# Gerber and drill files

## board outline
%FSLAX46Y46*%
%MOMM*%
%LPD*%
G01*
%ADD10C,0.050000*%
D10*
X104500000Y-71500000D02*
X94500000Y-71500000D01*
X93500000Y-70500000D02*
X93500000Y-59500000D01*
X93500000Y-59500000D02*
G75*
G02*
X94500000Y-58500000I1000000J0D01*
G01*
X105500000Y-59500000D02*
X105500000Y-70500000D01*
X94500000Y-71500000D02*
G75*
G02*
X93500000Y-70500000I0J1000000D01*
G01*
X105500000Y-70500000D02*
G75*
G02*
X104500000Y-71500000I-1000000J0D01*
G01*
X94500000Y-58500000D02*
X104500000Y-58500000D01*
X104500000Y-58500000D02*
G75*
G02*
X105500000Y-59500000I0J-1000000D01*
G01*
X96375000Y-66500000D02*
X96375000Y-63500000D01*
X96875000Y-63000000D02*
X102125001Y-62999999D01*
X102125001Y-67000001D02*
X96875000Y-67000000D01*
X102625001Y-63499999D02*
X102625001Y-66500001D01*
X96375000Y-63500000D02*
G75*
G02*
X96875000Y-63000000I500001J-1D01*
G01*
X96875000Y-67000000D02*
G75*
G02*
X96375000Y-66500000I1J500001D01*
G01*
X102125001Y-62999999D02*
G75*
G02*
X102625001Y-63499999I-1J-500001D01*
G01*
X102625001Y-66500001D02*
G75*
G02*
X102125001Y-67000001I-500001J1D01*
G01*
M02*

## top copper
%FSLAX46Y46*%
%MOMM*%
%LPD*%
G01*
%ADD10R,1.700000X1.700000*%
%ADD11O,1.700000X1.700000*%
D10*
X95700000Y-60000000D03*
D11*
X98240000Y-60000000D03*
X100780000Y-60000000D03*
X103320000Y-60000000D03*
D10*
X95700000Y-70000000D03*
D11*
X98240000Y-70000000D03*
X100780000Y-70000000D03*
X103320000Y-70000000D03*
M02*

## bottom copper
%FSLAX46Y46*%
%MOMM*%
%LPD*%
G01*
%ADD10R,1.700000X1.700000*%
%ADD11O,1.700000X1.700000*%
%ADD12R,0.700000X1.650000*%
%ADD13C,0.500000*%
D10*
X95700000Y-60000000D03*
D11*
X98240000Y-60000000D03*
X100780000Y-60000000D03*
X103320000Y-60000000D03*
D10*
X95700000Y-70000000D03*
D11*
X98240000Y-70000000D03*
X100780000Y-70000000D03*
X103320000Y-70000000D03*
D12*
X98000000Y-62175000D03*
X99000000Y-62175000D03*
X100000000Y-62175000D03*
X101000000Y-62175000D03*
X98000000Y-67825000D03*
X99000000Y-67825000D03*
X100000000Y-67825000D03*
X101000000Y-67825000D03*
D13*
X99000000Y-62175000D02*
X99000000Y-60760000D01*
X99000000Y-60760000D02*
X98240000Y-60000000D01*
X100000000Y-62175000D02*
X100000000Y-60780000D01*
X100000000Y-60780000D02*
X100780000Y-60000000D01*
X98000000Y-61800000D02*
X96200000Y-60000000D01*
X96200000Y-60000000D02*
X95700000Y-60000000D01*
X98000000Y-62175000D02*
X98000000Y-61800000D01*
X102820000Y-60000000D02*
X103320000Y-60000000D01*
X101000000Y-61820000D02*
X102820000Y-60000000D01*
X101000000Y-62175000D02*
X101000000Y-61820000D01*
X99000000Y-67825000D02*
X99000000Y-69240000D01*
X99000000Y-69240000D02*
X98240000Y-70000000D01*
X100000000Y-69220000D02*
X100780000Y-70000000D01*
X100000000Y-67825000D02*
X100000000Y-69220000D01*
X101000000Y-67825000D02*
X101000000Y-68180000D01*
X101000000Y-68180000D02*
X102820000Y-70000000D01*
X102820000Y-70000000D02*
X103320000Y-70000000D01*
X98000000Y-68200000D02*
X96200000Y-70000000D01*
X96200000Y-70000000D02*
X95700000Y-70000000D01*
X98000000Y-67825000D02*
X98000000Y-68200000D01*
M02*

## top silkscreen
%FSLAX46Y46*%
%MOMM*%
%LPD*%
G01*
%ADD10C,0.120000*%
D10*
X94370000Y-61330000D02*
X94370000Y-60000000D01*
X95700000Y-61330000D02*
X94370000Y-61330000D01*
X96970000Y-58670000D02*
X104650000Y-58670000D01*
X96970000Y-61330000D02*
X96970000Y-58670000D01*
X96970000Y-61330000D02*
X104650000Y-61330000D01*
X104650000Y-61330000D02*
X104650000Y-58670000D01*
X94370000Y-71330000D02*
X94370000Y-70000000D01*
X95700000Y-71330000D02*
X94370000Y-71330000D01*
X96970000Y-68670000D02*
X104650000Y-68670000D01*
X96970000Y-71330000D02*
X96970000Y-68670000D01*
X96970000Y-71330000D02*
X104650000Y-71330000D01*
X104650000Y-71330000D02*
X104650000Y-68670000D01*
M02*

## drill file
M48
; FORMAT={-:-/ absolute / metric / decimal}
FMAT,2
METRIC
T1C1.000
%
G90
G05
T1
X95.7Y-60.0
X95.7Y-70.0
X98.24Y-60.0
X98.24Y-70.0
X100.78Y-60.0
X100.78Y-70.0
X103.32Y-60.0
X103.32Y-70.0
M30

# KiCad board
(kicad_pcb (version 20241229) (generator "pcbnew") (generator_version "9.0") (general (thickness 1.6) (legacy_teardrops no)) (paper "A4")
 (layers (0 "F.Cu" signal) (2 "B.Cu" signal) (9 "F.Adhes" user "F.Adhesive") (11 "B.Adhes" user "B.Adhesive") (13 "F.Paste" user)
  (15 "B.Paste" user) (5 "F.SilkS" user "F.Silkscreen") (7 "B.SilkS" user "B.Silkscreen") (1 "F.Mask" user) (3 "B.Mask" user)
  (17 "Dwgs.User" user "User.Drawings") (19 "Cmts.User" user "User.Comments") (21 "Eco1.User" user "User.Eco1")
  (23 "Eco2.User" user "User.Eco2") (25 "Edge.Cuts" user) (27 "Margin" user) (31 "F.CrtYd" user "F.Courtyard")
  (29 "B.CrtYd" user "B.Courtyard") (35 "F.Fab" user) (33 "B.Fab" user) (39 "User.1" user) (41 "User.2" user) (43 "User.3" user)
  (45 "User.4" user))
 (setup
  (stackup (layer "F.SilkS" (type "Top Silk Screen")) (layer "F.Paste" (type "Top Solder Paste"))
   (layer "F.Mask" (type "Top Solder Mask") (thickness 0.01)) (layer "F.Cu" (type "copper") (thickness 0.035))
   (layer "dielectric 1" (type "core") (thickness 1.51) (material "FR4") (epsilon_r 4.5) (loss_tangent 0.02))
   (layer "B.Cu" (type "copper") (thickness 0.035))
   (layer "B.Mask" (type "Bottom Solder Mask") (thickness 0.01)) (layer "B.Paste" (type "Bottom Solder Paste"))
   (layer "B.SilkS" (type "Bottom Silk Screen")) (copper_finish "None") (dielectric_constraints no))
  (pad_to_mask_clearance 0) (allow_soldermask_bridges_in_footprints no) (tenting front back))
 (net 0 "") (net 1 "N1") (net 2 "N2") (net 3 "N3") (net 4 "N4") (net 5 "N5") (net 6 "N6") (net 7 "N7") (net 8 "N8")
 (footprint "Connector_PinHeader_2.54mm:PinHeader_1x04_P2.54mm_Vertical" (layer "F.Cu") (at 95.7 60 90)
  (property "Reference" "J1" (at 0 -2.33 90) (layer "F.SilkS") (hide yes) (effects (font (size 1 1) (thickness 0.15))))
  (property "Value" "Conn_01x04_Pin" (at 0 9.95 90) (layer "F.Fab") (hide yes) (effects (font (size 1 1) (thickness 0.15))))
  (fp_line (start -1.33 -1.33) (end 0 -1.33) (stroke (width 0.12) (type solid)) (layer "F.SilkS"))
  (fp_line (start -1.33 0) (end -1.33 -1.33) (stroke (width 0.12) (type solid)) (layer "F.SilkS"))
  (fp_line (start 1.33 1.27) (end 1.33 8.95) (stroke (width 0.12) (type solid)) (layer "F.SilkS"))
  (fp_line (start -1.33 1.27) (end 1.33 1.27) (stroke (width 0.12) (type solid)) (layer "F.SilkS"))
  (fp_line (start -1.33 1.27) (end -1.33 8.95) (stroke (width 0.12) (type solid)) (layer "F.SilkS"))
  (fp_line (start -1.33 8.95) (end 1.33 8.95) (stroke (width 0.12) (type solid)) (layer "F.SilkS"))
  (pad "1" thru_hole rect (at 0 0 90) (size 1.7 1.7) (drill 1) (layers "*.Cu" "*.Mask") (remove_unused_layers no) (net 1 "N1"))
  (pad "2" thru_hole oval (at 0 2.54 90) (size 1.7 1.7) (drill 1) (layers "*.Cu" "*.Mask") (remove_unused_layers no) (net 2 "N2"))
  (pad "3" thru_hole oval (at 0 5.08 90) (size 1.7 1.7) (drill 1) (layers "*.Cu" "*.Mask") (remove_unused_layers no) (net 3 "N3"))
  (pad "4" thru_hole oval (at 0 7.62 90) (size 1.7 1.7) (drill 1) (layers "*.Cu" "*.Mask") (remove_unused_layers no) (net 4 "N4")))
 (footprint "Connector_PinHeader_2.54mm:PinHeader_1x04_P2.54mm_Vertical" (layer "F.Cu") (at 95.7 70 90)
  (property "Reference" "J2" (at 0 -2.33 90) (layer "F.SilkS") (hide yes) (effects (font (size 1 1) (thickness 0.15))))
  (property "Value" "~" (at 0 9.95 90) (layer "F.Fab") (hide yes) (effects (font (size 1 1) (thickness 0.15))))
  (fp_line (start -1.33 -1.33) (end 0 -1.33) (stroke (width 0.12) (type solid)) (layer "F.SilkS"))
  (fp_line (start -1.33 0) (end -1.33 -1.33) (stroke (width 0.12) (type solid)) (layer "F.SilkS"))
  (fp_line (start 1.33 1.27) (end 1.33 8.95) (stroke (width 0.12) (type solid)) (layer "F.SilkS"))
  (fp_line (start -1.33 1.27) (end 1.33 1.27) (stroke (width 0.12) (type solid)) (layer "F.SilkS"))
  (fp_line (start -1.33 1.27) (end -1.33 8.95) (stroke (width 0.12) (type solid)) (layer "F.SilkS"))
  (fp_line (start -1.33 8.95) (end 1.33 8.95) (stroke (width 0.12) (type solid)) (layer "F.SilkS"))
  (pad "1" thru_hole rect (at 0 0 90) (size 1.7 1.7) (drill 1) (layers "*.Cu" "*.Mask") (remove_unused_layers no) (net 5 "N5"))
  (pad "2" thru_hole oval (at 0 2.54 90) (size 1.7 1.7) (drill 1) (layers "*.Cu" "*.Mask") (remove_unused_layers no) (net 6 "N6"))
  (pad "3" thru_hole oval (at 0 5.08 90) (size 1.7 1.7) (drill 1) (layers "*.Cu" "*.Mask") (remove_unused_layers no) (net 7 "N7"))
  (pad "4" thru_hole oval (at 0 7.62 90) (size 1.7 1.7) (drill 1) (layers "*.Cu" "*.Mask") (remove_unused_layers no) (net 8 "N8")))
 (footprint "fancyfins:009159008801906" (layer "B.Cu") (at 99.5 65)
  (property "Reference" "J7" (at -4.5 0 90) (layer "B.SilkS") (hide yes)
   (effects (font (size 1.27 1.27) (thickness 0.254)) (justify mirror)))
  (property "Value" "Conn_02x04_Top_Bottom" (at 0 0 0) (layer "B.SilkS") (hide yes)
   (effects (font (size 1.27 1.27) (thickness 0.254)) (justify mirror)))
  (fp_line (start -3.125 1.5) (end -3.125 -1.5) (stroke (width 0.05) (type default)) (layer "Edge.Cuts"))
  (fp_line (start -2.625 -2) (end 2.625001 -2.000001) (stroke (width 0.05) (type default)) (layer "Edge.Cuts"))
  (fp_line (start 2.625001 2.000001) (end -2.625 2) (stroke (width 0.05) (type default)) (layer "Edge.Cuts"))
  (fp_line (start 3.125001 -1.500001) (end 3.125001 1.500001) (stroke (width 0.05) (type default)) (layer "Edge.Cuts"))
  (fp_arc (start -3.125 -1.5) (mid -2.978553 -1.853553) (end -2.625 -2) (stroke (width 0.05) (type default)) (layer "Edge.Cuts"))
  (fp_arc (start -2.625 2) (mid -2.978553 1.853553) (end -3.125 1.5) (stroke (width 0.05) (type default)) (layer "Edge.Cuts"))
  (fp_arc (start 2.625001 -2.000001) (mid 2.978554 -1.853554) (end 3.125001 -1.500001) (stroke (width 0.05) (type default))
   (layer "Edge.Cuts"))
  (fp_arc (start 3.125001 1.500001) (mid 2.978554 1.853554) (end 2.625001 2.000001) (stroke (width 0.05) (type default)) (layer "Edge.Cuts"))
  (pad "1" smd rect (at -1.5 -2.825) (size 0.7 1.65) (layers "B.Cu" "B.Mask" "B.Paste") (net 1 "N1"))
  (pad "2" smd rect (at -0.5 -2.825) (size 0.7 1.65) (layers "B.Cu" "B.Mask" "B.Paste") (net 2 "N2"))
  (pad "3" smd rect (at 0.5 -2.825) (size 0.7 1.65) (layers "B.Cu" "B.Mask" "B.Paste") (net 3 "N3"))
  (pad "4" smd rect (at 1.5 -2.825) (size 0.7 1.65) (layers "B.Cu" "B.Mask" "B.Paste") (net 4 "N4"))
  (pad "5" smd rect (at -1.5 2.825) (size 0.7 1.65) (layers "B.Cu" "B.Mask" "B.Paste") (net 5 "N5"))
  (pad "6" smd rect (at -0.5 2.825) (size 0.7 1.65) (layers "B.Cu" "B.Mask" "B.Paste") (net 6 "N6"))
  (pad "7" smd rect (at 0.5 2.825) (size 0.7 1.65) (layers "B.Cu" "B.Mask" "B.Paste") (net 7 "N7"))
  (pad "8" smd rect (at 1.5 2.825) (size 0.7 1.65) (layers "B.Cu" "B.Mask" "B.Paste") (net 8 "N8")))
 (gr_line (start 104.5 71.5) (end 94.5 71.5) (stroke (width 0.05) (type default)) (layer "Edge.Cuts"))
 (gr_line (start 93.5 70.5) (end 93.5 59.5) (stroke (width 0.05) (type default)) (layer "Edge.Cuts"))
 (gr_arc (start 93.5 59.5) (mid 93.792893 58.792893) (end 94.5 58.5) (stroke (width 0.05) (type default)) (layer "Edge.Cuts"))
 (gr_line (start 105.5 59.5) (end 105.5 70.5) (stroke (width 0.05) (type default)) (layer "Edge.Cuts"))
 (gr_arc (start 94.5 71.5) (mid 93.792893 71.207107) (end 93.5 70.5) (stroke (width 0.05) (type default)) (layer "Edge.Cuts"))
 (gr_arc (start 105.5 70.5) (mid 105.207107 71.207107) (end 104.5 71.5) (stroke (width 0.05) (type default)) (layer "Edge.Cuts"))
 (gr_line (start 94.5 58.5) (end 104.5 58.5) (stroke (width 0.05) (type default)) (layer "Edge.Cuts"))
 (gr_arc (start 104.5 58.5) (mid 105.207107 58.792893) (end 105.5 59.5) (stroke (width 0.05) (type default)) (layer "Edge.Cuts"))
 (segment (start 99 62.175) (end 99 60.76) (width 0.5) (layer "B.Cu") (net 2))
 (segment (start 99 60.76) (end 98.24 60) (width 0.5) (layer "B.Cu") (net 2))
 (segment (start 100 62.175) (end 100 60.78) (width 0.5) (layer "B.Cu") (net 3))
 (segment (start 100 60.78) (end 100.78 60) (width 0.5) (layer "B.Cu") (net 3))
 (segment (start 98 61.8) (end 96.2 60) (width 0.5) (layer "B.Cu") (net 1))
 (segment (start 96.2 60) (end 95.7 60) (width 0.5) (layer "B.Cu") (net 1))
 (segment (start 98 62.175) (end 98 61.8) (width 0.5) (layer "B.Cu") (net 1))
 (segment (start 102.82 60) (end 103.32 60) (width 0.5) (layer "B.Cu") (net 4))
 (segment (start 101 61.82) (end 102.82 60) (width 0.5) (layer "B.Cu") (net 4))
 (segment (start 101 62.175) (end 101 61.82) (width 0.5) (layer "B.Cu") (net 4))
 (segment (start 99 67.825) (end 99 69.24) (width 0.5) (layer "B.Cu") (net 6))
 (segment (start 99 69.24) (end 98.24 70) (width 0.5) (layer "B.Cu") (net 6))
 (segment (start 100 69.22) (end 100.78 70) (width 0.5) (layer "B.Cu") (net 7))
 (segment (start 100 67.825) (end 100 69.22) (width 0.5) (layer "B.Cu") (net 7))
 (segment (start 101 67.825) (end 101 68.18) (width 0.5) (layer "B.Cu") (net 8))
 (segment (start 101 68.18) (end 102.82 70) (width 0.5) (layer "B.Cu") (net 8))
 (segment (start 102.82 70) (end 103.32 70) (width 0.5) (layer "B.Cu") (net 8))
 (segment (start 98 68.2) (end 96.2 70) (width 0.5) (layer "B.Cu") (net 5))
 (segment (start 96.2 70) (end 95.7 70) (width 0.5) (layer "B.Cu") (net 5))
 (segment (start 98 67.825) (end 98 68.2) (width 0.5) (layer "B.Cu") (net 5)))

